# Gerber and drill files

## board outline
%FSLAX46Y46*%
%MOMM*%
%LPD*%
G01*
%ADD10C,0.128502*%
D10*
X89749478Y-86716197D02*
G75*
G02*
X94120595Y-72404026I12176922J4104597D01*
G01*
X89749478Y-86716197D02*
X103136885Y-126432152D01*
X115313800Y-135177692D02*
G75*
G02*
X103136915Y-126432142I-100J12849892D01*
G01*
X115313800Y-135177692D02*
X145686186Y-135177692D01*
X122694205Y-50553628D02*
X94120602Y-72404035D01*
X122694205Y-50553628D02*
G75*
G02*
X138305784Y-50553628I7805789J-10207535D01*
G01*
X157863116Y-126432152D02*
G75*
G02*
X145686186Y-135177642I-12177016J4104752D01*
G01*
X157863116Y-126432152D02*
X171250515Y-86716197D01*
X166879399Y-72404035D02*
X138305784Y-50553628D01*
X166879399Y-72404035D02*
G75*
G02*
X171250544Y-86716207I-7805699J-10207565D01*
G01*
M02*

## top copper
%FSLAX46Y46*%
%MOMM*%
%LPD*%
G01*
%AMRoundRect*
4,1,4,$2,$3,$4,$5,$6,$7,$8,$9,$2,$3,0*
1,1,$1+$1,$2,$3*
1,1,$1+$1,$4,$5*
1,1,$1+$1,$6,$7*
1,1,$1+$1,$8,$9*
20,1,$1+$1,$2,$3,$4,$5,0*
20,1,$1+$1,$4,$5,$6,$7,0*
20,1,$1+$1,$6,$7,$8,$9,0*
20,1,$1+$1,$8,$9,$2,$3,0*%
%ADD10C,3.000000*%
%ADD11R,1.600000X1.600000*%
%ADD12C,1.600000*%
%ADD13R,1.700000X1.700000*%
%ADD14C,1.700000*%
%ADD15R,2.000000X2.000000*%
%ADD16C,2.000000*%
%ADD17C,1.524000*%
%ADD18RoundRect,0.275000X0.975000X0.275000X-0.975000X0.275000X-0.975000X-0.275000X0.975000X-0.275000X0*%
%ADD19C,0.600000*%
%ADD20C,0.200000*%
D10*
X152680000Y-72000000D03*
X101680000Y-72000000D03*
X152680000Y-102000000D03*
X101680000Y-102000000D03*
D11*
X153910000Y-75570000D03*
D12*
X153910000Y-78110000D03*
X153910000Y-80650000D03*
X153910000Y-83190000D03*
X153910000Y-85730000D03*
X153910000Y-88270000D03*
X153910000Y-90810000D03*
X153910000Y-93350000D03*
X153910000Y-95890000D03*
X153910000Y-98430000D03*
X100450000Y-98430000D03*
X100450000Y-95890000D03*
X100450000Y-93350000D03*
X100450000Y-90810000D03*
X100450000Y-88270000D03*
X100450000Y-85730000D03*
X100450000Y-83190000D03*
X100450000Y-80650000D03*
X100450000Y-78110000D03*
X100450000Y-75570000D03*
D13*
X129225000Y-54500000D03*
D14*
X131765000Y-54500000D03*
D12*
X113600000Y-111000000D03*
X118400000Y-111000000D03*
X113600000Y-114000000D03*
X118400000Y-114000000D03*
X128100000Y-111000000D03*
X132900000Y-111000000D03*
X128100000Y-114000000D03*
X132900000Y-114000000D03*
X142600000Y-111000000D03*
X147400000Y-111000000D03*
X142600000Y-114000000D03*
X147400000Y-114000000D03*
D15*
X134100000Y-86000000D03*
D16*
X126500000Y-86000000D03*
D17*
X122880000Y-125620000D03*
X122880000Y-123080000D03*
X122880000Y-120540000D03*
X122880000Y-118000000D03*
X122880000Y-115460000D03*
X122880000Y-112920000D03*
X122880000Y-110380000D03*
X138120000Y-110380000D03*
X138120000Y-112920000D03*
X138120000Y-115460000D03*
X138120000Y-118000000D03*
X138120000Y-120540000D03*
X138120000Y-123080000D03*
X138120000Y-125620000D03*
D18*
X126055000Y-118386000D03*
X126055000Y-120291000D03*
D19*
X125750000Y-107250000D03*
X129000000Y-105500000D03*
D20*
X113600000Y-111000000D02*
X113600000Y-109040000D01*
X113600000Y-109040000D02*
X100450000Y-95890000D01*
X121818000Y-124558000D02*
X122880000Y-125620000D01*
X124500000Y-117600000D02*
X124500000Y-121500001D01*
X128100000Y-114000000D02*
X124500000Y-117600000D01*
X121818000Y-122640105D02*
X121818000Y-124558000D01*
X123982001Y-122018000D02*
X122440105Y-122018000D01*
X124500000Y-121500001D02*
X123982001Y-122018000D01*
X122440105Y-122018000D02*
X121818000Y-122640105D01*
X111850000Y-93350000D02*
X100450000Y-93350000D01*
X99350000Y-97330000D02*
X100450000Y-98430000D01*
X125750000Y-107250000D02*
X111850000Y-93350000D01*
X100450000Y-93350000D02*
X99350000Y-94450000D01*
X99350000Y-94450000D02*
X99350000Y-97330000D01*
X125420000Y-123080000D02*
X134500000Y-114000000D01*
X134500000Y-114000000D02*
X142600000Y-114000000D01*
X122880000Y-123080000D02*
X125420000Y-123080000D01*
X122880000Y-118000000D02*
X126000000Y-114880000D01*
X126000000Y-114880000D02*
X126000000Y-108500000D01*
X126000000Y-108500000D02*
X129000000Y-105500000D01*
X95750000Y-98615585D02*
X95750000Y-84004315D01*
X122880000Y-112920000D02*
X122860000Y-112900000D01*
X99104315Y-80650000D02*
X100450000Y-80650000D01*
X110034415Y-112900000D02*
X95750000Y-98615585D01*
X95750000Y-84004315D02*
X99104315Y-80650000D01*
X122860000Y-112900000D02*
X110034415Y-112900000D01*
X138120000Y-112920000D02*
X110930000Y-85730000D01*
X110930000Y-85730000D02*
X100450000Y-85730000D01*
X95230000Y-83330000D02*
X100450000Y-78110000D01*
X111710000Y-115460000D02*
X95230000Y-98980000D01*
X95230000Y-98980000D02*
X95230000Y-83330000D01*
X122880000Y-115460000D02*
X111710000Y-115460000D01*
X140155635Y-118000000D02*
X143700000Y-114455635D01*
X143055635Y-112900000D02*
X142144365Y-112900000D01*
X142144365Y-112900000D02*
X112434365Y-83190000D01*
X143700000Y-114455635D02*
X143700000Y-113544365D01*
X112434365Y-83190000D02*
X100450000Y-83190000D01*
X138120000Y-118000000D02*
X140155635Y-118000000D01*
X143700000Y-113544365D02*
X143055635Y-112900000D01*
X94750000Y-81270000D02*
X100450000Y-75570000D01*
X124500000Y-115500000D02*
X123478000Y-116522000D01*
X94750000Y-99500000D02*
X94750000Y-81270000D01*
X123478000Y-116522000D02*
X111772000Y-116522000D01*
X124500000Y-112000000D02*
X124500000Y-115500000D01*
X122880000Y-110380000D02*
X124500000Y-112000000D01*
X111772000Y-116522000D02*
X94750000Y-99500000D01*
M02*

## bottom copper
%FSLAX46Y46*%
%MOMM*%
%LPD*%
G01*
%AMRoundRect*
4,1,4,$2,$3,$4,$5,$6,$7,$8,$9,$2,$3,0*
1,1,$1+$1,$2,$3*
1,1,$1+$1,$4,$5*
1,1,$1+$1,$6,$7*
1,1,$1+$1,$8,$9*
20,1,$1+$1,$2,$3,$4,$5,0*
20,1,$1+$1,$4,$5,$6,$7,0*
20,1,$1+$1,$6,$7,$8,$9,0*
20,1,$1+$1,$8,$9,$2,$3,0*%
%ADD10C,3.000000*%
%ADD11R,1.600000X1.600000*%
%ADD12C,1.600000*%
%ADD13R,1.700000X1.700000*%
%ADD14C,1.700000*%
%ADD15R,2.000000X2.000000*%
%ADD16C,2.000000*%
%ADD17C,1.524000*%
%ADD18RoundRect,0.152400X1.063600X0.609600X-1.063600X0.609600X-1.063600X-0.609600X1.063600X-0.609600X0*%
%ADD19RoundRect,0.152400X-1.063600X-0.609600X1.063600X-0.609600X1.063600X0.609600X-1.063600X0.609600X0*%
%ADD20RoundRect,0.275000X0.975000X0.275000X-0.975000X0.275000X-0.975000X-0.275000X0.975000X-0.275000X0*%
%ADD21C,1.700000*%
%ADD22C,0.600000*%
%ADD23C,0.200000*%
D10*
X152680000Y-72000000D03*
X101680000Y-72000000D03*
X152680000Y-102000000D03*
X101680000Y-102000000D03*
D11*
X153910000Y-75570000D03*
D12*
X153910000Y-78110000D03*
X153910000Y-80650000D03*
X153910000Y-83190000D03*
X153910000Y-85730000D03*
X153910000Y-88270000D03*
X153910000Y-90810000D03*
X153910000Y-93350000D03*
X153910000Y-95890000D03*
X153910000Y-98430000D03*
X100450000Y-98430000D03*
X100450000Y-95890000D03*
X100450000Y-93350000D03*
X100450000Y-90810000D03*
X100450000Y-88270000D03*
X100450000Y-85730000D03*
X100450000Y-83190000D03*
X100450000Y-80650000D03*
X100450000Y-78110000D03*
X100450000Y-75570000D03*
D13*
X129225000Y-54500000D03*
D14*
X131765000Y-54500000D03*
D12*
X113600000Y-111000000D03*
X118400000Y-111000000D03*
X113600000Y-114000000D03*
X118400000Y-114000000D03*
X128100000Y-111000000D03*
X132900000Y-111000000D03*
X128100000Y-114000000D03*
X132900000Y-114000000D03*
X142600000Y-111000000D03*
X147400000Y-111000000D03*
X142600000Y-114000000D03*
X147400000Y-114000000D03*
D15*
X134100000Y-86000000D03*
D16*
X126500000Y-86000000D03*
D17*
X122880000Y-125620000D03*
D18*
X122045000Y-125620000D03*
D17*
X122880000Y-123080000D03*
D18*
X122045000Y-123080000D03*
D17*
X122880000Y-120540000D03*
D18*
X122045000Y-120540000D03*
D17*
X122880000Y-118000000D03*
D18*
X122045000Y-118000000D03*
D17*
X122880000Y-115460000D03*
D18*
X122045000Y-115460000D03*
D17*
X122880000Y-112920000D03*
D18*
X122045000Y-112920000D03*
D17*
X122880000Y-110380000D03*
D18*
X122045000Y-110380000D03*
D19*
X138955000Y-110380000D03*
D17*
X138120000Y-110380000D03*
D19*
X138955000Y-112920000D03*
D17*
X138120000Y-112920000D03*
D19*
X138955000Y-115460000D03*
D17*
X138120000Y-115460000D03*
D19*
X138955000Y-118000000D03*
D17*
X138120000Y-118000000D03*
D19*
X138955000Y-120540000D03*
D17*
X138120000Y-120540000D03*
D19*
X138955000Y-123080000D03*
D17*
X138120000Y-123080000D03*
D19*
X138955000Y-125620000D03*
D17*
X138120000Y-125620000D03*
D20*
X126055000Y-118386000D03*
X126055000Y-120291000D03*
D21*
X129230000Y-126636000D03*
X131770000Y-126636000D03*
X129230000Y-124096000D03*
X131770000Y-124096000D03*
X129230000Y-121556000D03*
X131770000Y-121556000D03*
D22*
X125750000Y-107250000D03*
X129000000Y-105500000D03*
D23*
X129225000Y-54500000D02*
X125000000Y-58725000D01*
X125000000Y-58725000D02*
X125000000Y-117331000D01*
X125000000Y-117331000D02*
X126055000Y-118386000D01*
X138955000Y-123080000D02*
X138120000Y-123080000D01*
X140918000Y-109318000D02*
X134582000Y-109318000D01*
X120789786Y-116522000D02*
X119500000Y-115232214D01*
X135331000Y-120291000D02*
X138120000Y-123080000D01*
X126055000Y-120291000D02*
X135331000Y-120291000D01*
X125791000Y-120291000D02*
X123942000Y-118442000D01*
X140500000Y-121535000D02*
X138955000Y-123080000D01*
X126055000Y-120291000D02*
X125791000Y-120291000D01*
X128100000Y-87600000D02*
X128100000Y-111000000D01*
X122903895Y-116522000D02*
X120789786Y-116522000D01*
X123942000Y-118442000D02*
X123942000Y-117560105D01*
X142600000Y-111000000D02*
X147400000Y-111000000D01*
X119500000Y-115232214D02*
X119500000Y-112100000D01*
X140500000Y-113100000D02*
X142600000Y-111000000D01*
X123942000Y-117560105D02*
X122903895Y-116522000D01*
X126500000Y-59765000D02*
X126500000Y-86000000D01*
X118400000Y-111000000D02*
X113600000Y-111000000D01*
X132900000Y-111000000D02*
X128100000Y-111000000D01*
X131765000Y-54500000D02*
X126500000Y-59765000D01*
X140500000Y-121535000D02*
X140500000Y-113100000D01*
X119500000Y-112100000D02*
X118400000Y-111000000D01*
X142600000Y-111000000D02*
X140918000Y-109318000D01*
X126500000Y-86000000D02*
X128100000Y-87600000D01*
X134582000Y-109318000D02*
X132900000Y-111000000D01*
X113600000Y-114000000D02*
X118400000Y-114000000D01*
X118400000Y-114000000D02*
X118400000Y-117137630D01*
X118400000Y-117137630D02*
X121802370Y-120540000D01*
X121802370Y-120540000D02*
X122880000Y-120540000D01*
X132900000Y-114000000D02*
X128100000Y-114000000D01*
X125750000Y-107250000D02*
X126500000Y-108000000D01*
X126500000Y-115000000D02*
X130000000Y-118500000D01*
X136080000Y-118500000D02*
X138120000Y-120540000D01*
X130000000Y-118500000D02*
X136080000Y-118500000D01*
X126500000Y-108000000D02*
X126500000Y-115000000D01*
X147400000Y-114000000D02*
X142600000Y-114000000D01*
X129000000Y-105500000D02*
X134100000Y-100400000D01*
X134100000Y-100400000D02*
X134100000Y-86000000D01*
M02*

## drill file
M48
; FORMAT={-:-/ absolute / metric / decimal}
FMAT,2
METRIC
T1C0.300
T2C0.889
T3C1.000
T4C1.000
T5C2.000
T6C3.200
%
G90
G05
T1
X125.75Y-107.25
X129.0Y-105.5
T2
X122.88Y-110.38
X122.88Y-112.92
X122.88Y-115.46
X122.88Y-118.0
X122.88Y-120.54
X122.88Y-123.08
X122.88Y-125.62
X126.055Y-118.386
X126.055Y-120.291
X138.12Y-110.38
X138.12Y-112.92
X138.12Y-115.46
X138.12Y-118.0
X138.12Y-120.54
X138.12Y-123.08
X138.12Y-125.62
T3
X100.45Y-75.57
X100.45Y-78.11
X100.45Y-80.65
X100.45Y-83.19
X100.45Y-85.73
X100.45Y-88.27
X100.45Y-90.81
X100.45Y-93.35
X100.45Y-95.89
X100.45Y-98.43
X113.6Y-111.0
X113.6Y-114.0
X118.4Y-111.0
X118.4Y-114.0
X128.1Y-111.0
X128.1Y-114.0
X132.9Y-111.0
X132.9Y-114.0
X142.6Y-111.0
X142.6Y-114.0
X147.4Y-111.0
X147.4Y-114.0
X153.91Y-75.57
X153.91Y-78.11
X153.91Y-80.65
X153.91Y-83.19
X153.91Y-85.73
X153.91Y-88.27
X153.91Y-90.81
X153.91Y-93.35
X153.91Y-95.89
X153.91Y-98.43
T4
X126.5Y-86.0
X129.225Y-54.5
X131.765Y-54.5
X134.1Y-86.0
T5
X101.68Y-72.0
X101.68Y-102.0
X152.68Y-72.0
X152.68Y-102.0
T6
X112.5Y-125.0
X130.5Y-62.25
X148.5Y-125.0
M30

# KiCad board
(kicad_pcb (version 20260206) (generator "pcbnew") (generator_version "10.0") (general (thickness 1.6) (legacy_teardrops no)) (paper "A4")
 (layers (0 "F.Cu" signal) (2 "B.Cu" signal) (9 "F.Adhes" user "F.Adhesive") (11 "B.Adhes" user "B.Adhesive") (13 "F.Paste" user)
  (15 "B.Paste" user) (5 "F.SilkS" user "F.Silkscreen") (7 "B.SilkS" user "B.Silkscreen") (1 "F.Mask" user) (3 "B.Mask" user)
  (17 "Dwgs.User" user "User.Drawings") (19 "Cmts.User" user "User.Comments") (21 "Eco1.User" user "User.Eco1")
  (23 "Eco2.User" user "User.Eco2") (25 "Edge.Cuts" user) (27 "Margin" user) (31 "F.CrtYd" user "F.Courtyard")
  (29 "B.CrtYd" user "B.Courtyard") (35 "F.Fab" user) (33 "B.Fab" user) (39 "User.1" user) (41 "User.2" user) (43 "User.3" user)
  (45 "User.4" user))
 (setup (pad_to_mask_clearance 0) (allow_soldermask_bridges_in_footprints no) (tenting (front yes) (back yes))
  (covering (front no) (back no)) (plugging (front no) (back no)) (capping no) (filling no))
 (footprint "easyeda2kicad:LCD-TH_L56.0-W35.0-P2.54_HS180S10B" (layer "F.Cu") (at 127.18 87 -90)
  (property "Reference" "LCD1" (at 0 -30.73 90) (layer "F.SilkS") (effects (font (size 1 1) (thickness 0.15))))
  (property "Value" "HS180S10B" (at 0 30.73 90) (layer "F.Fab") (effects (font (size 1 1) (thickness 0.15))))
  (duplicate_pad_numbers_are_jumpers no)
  (pad "" thru_hole circle (at -15 -25.5 270) (size 3 3) (drill 2) (layers "*.Cu" "*.Mask") (remove_unused_layers no))
  (pad "" thru_hole circle (at -15 25.5 270) (size 3 3) (drill 2) (layers "*.Cu" "*.Mask") (remove_unused_layers no))
  (pad "" thru_hole circle (at 15 -25.5 270) (size 3 3) (drill 2) (layers "*.Cu" "*.Mask") (remove_unused_layers no))
  (pad "" thru_hole circle (at 15 25.5 270) (size 3 3) (drill 2) (layers "*.Cu" "*.Mask") (remove_unused_layers no))
  (pad "1" thru_hole rect (at -11.43 -26.73 270) (size 1.6 1.6) (drill 0.999998) (layers "*.Cu" "*.Mask") (remove_unused_layers no)
   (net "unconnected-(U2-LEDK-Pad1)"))
  (pad "2" thru_hole circle (at -8.89 -26.73 270) (size 1.6 1.6) (drill 0.999998) (layers "*.Cu" "*.Mask") (remove_unused_layers no)
   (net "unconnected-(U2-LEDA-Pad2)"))
  (pad "3" thru_hole circle (at -6.35 -26.73 270) (size 1.6 1.6) (drill 0.999998) (layers "*.Cu" "*.Mask") (remove_unused_layers no)
   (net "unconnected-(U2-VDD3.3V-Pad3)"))
  (pad "4" thru_hole circle (at -3.81 -26.73 270) (size 1.6 1.6) (drill 0.999998) (layers "*.Cu" "*.Mask") (remove_unused_layers no)
   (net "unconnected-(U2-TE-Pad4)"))
  (pad "5" thru_hole circle (at -1.27 -26.73 270) (size 1.6 1.6) (drill 0.999998) (layers "*.Cu" "*.Mask") (remove_unused_layers no)
   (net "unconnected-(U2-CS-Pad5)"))
  (pad "6" thru_hole circle (at 1.27 -26.73 270) (size 1.6 1.6) (drill 0.999998) (layers "*.Cu" "*.Mask") (remove_unused_layers no)
   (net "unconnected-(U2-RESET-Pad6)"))
  (pad "7" thru_hole circle (at 3.81 -26.73 270) (size 1.6 1.6) (drill 0.999998) (layers "*.Cu" "*.Mask") (remove_unused_layers no)
   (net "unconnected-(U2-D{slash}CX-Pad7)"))
  (pad "8" thru_hole circle (at 6.35 -26.73 270) (size 1.6 1.6) (drill 0.999998) (layers "*.Cu" "*.Mask") (remove_unused_layers no)
   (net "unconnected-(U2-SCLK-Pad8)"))
  (pad "9" thru_hole circle (at 8.89 -26.73 270) (size 1.6 1.6) (drill 0.999998) (layers "*.Cu" "*.Mask") (remove_unused_layers no)
   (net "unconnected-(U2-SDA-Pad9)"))
  (pad "10" thru_hole circle (at 11.43 -26.73 270) (size 1.6 1.6) (drill 0.999998) (layers "*.Cu" "*.Mask") (remove_unused_layers no)
   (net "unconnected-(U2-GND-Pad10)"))
  (pad "11" thru_hole circle (at 11.43 26.73 270) (size 1.6 1.6) (drill 0.999998) (layers "*.Cu" "*.Mask") (remove_unused_layers no)
   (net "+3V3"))
  (pad "12" thru_hole circle (at 8.89 26.73 270) (size 1.6 1.6) (drill 0.999998) (layers "*.Cu" "*.Mask") (remove_unused_layers no)
   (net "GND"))
  (pad "13" thru_hole circle (at 6.35 26.73 270) (size 1.6 1.6) (drill 0.999998) (layers "*.Cu" "*.Mask") (remove_unused_layers no)
   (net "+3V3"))
  (pad "14" thru_hole circle (at 3.81 26.73 270) (size 1.6 1.6) (drill 0.999998) (layers "*.Cu" "*.Mask") (remove_unused_layers no))
  (pad "15" thru_hole circle (at 1.27 26.73 270) (size 1.6 1.6) (drill 0.999998) (layers "*.Cu" "*.Mask") (remove_unused_layers no))
  (pad "16" thru_hole circle (at -1.27 26.73 270) (size 1.6 1.6) (drill 0.999998) (layers "*.Cu" "*.Mask") (remove_unused_layers no)
   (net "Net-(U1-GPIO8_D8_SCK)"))
  (pad "17" thru_hole circle (at -3.81 26.73 270) (size 1.6 1.6) (drill 0.999998) (layers "*.Cu" "*.Mask") (remove_unused_layers no)
   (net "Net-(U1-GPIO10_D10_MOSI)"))
  (pad "18" thru_hole circle (at -6.35 26.73 270) (size 1.6 1.6) (drill 0.999998) (layers "*.Cu" "*.Mask") (remove_unused_layers no)
   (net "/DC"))
  (pad "19" thru_hole circle (at -8.89 26.73 270) (size 1.6 1.6) (drill 0.999998) (layers "*.Cu" "*.Mask") (remove_unused_layers no)
   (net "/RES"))
  (pad "20" thru_hole circle (at -11.43 26.73 270) (size 1.6 1.6) (drill 0.999998) (layers "*.Cu" "*.Mask") (remove_unused_layers no)
   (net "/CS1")))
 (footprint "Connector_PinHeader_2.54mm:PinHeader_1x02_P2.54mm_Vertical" (layer "F.Cu") (at 129.225 54.5 90)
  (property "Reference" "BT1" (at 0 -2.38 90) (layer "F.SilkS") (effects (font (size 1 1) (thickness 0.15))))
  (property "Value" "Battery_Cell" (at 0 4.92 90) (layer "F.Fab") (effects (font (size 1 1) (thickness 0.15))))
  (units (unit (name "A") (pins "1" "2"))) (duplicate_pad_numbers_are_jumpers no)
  (pad "1" thru_hole rect (at 0 0 90) (size 1.7 1.7) (drill 1) (layers "*.Cu" "*.Mask") (remove_unused_layers no) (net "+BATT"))
  (pad "2" thru_hole circle (at 0 2.54 90) (size 1.7 1.7) (drill 1) (layers "*.Cu" "*.Mask") (remove_unused_layers no) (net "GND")))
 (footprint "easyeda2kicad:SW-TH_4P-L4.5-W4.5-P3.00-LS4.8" (layer "F.Cu") (at 116 112.5)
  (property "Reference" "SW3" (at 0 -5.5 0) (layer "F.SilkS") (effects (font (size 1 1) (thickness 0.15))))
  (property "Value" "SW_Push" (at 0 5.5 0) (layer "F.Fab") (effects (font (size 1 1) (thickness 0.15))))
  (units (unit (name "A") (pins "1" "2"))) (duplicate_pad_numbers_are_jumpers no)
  (pad "1" thru_hole circle (at -2.4 -1.5) (size 1.6 1.6) (drill 0.999998) (layers "*.Cu" "*.Mask") (remove_unused_layers no) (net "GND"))
  (pad "1" thru_hole circle (at 2.4 -1.5) (size 1.6 1.6) (drill 0.999998) (layers "*.Cu" "*.Mask") (remove_unused_layers no) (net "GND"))
  (pad "2" thru_hole circle (at -2.4 1.5) (size 1.6 1.6) (drill 0.999998) (layers "*.Cu" "*.Mask") (remove_unused_layers no)
   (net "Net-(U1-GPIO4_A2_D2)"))
  (pad "2" thru_hole circle (at 2.4 1.5) (size 1.6 1.6) (drill 0.999998) (layers "*.Cu" "*.Mask") (remove_unused_layers no)
   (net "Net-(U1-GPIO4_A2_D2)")))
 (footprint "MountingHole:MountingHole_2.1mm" (layer "F.Cu") (at 148.5 125)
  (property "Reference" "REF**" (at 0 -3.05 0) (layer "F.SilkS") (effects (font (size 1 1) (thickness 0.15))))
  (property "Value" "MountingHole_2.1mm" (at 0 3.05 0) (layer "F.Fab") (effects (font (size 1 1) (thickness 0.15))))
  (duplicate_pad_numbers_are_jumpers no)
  (pad "" np_thru_hole circle (at 0 0) (size 3.2 3.2) (drill 3.2) (layers "*.Cu" "*.Mask")))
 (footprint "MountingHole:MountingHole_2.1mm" (layer "F.Cu") (at 112.5 125)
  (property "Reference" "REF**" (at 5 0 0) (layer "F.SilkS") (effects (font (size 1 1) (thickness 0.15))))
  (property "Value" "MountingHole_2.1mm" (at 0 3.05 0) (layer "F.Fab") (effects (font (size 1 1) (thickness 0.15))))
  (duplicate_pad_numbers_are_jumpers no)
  (pad "" np_thru_hole circle (at 0 0) (size 3.2 3.2) (drill 3.2) (layers "*.Cu" "*.Mask")))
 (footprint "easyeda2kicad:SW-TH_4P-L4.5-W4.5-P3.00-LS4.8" (layer "F.Cu") (at 130.5 112.5)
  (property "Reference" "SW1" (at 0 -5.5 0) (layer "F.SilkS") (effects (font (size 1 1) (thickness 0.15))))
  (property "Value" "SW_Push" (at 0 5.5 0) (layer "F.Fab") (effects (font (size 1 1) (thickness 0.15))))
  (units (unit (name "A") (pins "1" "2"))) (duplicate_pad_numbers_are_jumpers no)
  (pad "1" thru_hole circle (at -2.4 -1.5) (size 1.6 1.6) (drill 0.999998) (layers "*.Cu" "*.Mask") (remove_unused_layers no) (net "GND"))
  (pad "1" thru_hole circle (at 2.4 -1.5) (size 1.6 1.6) (drill 0.999998) (layers "*.Cu" "*.Mask") (remove_unused_layers no) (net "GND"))
  (pad "2" thru_hole circle (at -2.4 1.5) (size 1.6 1.6) (drill 0.999998) (layers "*.Cu" "*.Mask") (remove_unused_layers no)
   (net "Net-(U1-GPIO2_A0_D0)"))
  (pad "2" thru_hole circle (at 2.4 1.5) (size 1.6 1.6) (drill 0.999998) (layers "*.Cu" "*.Mask") (remove_unused_layers no)
   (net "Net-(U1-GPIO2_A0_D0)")))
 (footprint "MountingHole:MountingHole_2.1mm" (layer "F.Cu") (at 130.5 62.25)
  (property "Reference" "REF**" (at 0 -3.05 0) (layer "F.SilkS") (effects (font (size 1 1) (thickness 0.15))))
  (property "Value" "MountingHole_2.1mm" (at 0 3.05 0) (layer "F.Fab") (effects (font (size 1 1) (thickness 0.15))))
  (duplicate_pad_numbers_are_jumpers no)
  (pad "" np_thru_hole circle (at 0 0) (size 3.2 3.2) (drill 3.2) (layers "*.Cu" "*.Mask")))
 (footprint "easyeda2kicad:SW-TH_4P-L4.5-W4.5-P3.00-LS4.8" (layer "F.Cu") (at 145 112.5)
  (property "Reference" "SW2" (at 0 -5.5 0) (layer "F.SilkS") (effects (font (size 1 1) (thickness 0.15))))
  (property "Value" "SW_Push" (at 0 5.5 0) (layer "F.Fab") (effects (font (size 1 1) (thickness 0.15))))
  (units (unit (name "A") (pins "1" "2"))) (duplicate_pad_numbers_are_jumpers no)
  (pad "1" thru_hole circle (at -2.4 -1.5) (size 1.6 1.6) (drill 0.999998) (layers "*.Cu" "*.Mask") (remove_unused_layers no) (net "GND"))
  (pad "1" thru_hole circle (at 2.4 -1.5) (size 1.6 1.6) (drill 0.999998) (layers "*.Cu" "*.Mask") (remove_unused_layers no) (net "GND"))
  (pad "2" thru_hole circle (at -2.4 1.5) (size 1.6 1.6) (drill 0.999998) (layers "*.Cu" "*.Mask") (remove_unused_layers no)
   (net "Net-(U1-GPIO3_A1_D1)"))
  (pad "2" thru_hole circle (at 2.4 1.5) (size 1.6 1.6) (drill 0.999998) (layers "*.Cu" "*.Mask") (remove_unused_layers no)
   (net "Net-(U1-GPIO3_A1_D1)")))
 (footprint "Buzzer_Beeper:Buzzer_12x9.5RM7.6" (layer "B.Cu") (at 134.1 86 180)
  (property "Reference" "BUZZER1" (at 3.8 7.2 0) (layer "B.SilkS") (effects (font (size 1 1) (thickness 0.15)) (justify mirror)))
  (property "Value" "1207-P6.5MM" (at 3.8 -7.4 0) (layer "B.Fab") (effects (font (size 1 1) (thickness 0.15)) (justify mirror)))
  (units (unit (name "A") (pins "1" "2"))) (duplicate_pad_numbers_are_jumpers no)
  (pad "1" thru_hole rect (at 0 0 180) (size 2 2) (drill 1) (layers "*.Cu" "*.Mask") (remove_unused_layers no) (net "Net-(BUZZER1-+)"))
  (pad "2" thru_hole circle (at 7.6 0 180) (size 2 2) (drill 1) (layers "*.Cu" "*.Mask") (remove_unused_layers no) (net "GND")))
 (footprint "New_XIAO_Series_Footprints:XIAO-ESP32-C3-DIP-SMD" (layer "B.Cu") (at 130.5 118 -90)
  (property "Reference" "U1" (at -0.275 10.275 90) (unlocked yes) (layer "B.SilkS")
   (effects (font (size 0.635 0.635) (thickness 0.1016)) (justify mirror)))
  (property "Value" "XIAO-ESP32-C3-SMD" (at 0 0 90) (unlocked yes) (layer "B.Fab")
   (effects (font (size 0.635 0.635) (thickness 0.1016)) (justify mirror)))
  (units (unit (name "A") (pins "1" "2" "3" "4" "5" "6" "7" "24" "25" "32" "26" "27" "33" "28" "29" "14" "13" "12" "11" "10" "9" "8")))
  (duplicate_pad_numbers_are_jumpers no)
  (pad "1" thru_hole circle (at 7.62 7.62 180) (size 1.524 1.524) (drill 0.889) (layers "*.Cu" "*.Mask") (remove_unused_layers no)
   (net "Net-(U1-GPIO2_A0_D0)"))
  (pad "1" smd roundrect (at 7.62 8.455 180) (size 2.432 1.524) (layers "B.Cu" "B.Mask") (roundrect_rratio 0.1) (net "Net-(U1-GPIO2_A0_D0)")
   (thermal_bridge_angle 45))
  (pad "2" thru_hole circle (at 5.08 7.62 180) (size 1.524 1.524) (drill 0.889) (layers "*.Cu" "*.Mask") (remove_unused_layers no)
   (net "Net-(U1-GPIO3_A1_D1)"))
  (pad "2" smd roundrect (at 5.08 8.455 180) (size 2.432 1.524) (layers "B.Cu" "B.Mask") (roundrect_rratio 0.1) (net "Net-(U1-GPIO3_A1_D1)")
   (thermal_bridge_angle 45))
  (pad "3" thru_hole circle (at 2.54 7.62 180) (size 1.524 1.524) (drill 0.889) (layers "*.Cu" "*.Mask") (remove_unused_layers no)
   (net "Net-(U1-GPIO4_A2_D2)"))
  (pad "3" smd roundrect (at 2.54 8.455 180) (size 2.432 1.524) (layers "B.Cu" "B.Mask") (roundrect_rratio 0.1) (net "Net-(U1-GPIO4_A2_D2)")
   (thermal_bridge_angle 45))
  (pad "4" thru_hole circle (at 0 7.62 180) (size 1.524 1.524) (drill 0.889) (layers "*.Cu" "*.Mask") (remove_unused_layers no)
   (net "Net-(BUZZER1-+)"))
  (pad "4" smd roundrect (at 0 8.455 180) (size 2.432 1.524) (layers "B.Cu" "B.Mask") (roundrect_rratio 0.1) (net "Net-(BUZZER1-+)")
   (thermal_bridge_angle 45))
  (pad "5" thru_hole circle (at -2.54 7.62 180) (size 1.524 1.524) (drill 0.889) (layers "*.Cu" "*.Mask") (remove_unused_layers no)
   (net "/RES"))
  (pad "5" smd roundrect (at -2.54 8.455 180) (size 2.432 1.524) (layers "B.Cu" "B.Mask") (roundrect_rratio 0.1) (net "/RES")
   (thermal_bridge_angle 45))
  (pad "6" thru_hole circle (at -5.08 7.62 180) (size 1.524 1.524) (drill 0.889) (layers "*.Cu" "*.Mask") (remove_unused_layers no)
   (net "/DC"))
  (pad "6" smd roundrect (at -5.08 8.455 180) (size 2.432 1.524) (layers "B.Cu" "B.Mask") (roundrect_rratio 0.1) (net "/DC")
   (thermal_bridge_angle 45))
  (pad "7" thru_hole circle (at -7.62 7.62 180) (size 1.524 1.524) (drill 0.889) (layers "*.Cu" "*.Mask") (remove_unused_layers no)
   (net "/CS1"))
  (pad "7" smd roundrect (at -7.62 8.455 180) (size 2.432 1.524) (layers "B.Cu" "B.Mask") (roundrect_rratio 0.1) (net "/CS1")
   (thermal_bridge_angle 45))
  (pad "8" smd roundrect (at -7.62 -8.455) (size 2.432 1.524) (layers "B.Cu" "B.Mask") (roundrect_rratio 0.1)
   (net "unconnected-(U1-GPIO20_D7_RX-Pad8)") (thermal_bridge_angle 45))
  (pad "8" thru_hole circle (at -7.62 -7.62) (size 1.524 1.524) (drill 0.889) (layers "*.Cu" "*.Mask") (remove_unused_layers no)
   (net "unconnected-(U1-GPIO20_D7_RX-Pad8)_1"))
  (pad "9" smd roundrect (at -5.08 -8.455) (size 2.432 1.524) (layers "B.Cu" "B.Mask") (roundrect_rratio 0.1) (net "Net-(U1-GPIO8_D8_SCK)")
   (thermal_bridge_angle 45))
  (pad "9" thru_hole circle (at -5.08 -7.62) (size 1.524 1.524) (drill 0.889) (layers "*.Cu" "*.Mask") (remove_unused_layers no)
   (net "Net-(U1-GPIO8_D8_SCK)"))
  (pad "10" smd roundrect (at -2.54 -8.455) (size 2.432 1.524) (layers "B.Cu" "B.Mask") (roundrect_rratio 0.1)
   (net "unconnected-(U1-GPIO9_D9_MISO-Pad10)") (thermal_bridge_angle 45))
  (pad "10" thru_hole circle (at -2.54 -7.62) (size 1.524 1.524) (drill 0.889) (layers "*.Cu" "*.Mask") (remove_unused_layers no)
   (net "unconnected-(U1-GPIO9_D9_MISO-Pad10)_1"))
  (pad "11" smd roundrect (at 0 -8.455) (size 2.432 1.524) (layers "B.Cu" "B.Mask") (roundrect_rratio 0.1) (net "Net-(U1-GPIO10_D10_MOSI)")
   (thermal_bridge_angle 45))
  (pad "11" thru_hole circle (at 0 -7.62) (size 1.524 1.524) (drill 0.889) (layers "*.Cu" "*.Mask") (remove_unused_layers no)
   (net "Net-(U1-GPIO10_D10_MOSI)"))
  (pad "12" smd roundrect (at 2.54 -8.455) (size 2.432 1.524) (layers "B.Cu" "B.Mask") (roundrect_rratio 0.1) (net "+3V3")
   (thermal_bridge_angle 45))
  (pad "12" thru_hole circle (at 2.54 -7.62) (size 1.524 1.524) (drill 0.889) (layers "*.Cu" "*.Mask") (remove_unused_layers no)
   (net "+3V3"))
  (pad "13" smd roundrect (at 5.08 -8.455) (size 2.432 1.524) (layers "B.Cu" "B.Mask") (roundrect_rratio 0.1) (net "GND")
   (thermal_bridge_angle 45))
  (pad "13" thru_hole circle (at 5.08 -7.62) (size 1.524 1.524) (drill 0.889) (layers "*.Cu" "*.Mask") (remove_unused_layers no) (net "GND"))
  (pad "14" smd roundrect (at 7.62 -8.455) (size 2.432 1.524) (layers "B.Cu" "B.Mask") (roundrect_rratio 0.1) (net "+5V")
   (thermal_bridge_angle 45))
  (pad "14" thru_hole circle (at 7.62 -7.62) (size 1.524 1.524) (drill 0.889) (layers "*.Cu" "*.Mask") (remove_unused_layers no) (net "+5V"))
  (pad "15" thru_hole roundrect (at 0.386 4.445 180) (size 2.5 1.1) (drill 0.889) (layers "*.Cu" "*.Mask") (remove_unused_layers no)
   (roundrect_rratio 0.25) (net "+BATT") (thermal_bridge_angle 45))
  (pad "16" thru_hole roundrect (at 2.291 4.445 180) (size 2.5 1.1) (drill 0.889) (layers "*.Cu" "*.Mask") (remove_unused_layers no)
   (roundrect_rratio 0.25) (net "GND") (thermal_bridge_angle 45))
  (pad "17" smd circle (at 8.636 1.27) (size 1.7 1.7) (layers "B.Cu" "B.Mask" "B.Paste"))
  (pad "18" smd circle (at 8.636 -1.27) (size 1.7 1.7) (layers "B.Cu" "B.Mask" "B.Paste"))
  (pad "19" smd circle (at 6.096 1.27) (size 1.7 1.7) (layers "B.Cu" "B.Mask" "B.Paste"))
  (pad "20" smd circle (at 6.096 -1.27) (size 1.7 1.7) (layers "B.Cu" "B.Mask" "B.Paste"))
  (pad "21" smd circle (at 3.556 1.27) (size 1.7 1.7) (layers "B.Cu" "B.Mask" "B.Paste"))
  (pad "22" smd circle (at 3.556 -1.27) (size 1.7 1.7) (layers "B.Cu" "B.Mask" "B.Paste")))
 (gr_arc (start 89.749478 86.716197) (mid 89.636692 78.858169) (end 94.120602 72.404035) (stroke (width 0.128502) (type default))
  (layer "Edge.Cuts"))
 (gr_line (start 89.749478 86.716197) (end 103.136885 126.432152) (stroke (width 0.128502) (type default)) (layer "Edge.Cuts"))
 (gr_arc (start 115.3138 135.177692) (mid 107.817744 132.764785) (end 103.136885 126.432152) (stroke (width 0.128502) (type default))
  (layer "Edge.Cuts"))
 (gr_line (start 115.3138 135.177692) (end 145.686186 135.177692) (stroke (width 0.128502) (type default)) (layer "Edge.Cuts"))
 (gr_line (start 122.694205 50.553628) (end 94.120602 72.404035) (stroke (width 0.128502) (type default)) (layer "Edge.Cuts"))
 (gr_arc (start 122.694205 50.553628) (mid 130.499996 47.9111) (end 138.305784 50.553628) (stroke (width 0.128502) (type default))
  (layer "Edge.Cuts"))
 (gr_arc (start 157.863116 126.432152) (mid 153.182199 132.764729) (end 145.686186 135.177692) (stroke (width 0.128502) (type default))
  (layer "Edge.Cuts"))
 (gr_line (start 157.863116 126.432152) (end 171.250515 86.716197) (stroke (width 0.128502) (type default)) (layer "Edge.Cuts"))
 (gr_line (start 166.879399 72.404035) (end 138.305784 50.553628) (stroke (width 0.128502) (type default)) (layer "Edge.Cuts"))
 (gr_arc (start 166.879399 72.404035) (mid 171.363322 78.858174) (end 171.250515 86.716197) (stroke (width 0.128502) (type default))
  (layer "Edge.Cuts"))
 (segment (start 129.225 54.5) (end 125 58.725) (width 0.2) (layer "B.Cu") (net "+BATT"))
 (segment (start 125 58.725) (end 125 117.331) (width 0.2) (layer "B.Cu") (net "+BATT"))
 (segment (start 125 117.331) (end 126.055 118.386) (width 0.2) (layer "B.Cu") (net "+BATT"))
 (segment (start 113.6 111) (end 113.6 109.04) (width 0.2) (layer "F.Cu") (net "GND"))
 (segment (start 113.6 109.04) (end 100.45 95.89) (width 0.2) (layer "F.Cu") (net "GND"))
 (segment (start 138.955 123.08) (end 138.12 123.08) (width 0.2) (layer "B.Cu") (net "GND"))
 (segment (start 140.918 109.318) (end 134.582 109.318) (width 0.2) (layer "B.Cu") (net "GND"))
 (segment (start 120.789786 116.522) (end 119.5 115.232214) (width 0.2) (layer "B.Cu") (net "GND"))
 (segment (start 135.331 120.291) (end 138.12 123.08) (width 0.2) (layer "B.Cu") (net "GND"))
 (segment (start 126.055 120.291) (end 135.331 120.291) (width 0.2) (layer "B.Cu") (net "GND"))
 (segment (start 125.791 120.291) (end 123.942 118.442) (width 0.2) (layer "B.Cu") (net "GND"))
 (segment (start 140.5 121.535) (end 138.955 123.08) (width 0.2) (layer "B.Cu") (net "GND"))
 (segment (start 126.055 120.291) (end 125.791 120.291) (width 0.2) (layer "B.Cu") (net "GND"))
 (segment (start 128.1 87.6) (end 128.1 111) (width 0.2) (layer "B.Cu") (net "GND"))
 (segment (start 122.903895 116.522) (end 120.789786 116.522) (width 0.2) (layer "B.Cu") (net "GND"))
 (segment (start 123.942 118.442) (end 123.942 117.560105) (width 0.2) (layer "B.Cu") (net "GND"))
 (segment (start 142.6 111) (end 147.4 111) (width 0.2) (layer "B.Cu") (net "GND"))
 (segment (start 119.5 115.232214) (end 119.5 112.1) (width 0.2) (layer "B.Cu") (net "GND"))
 (segment (start 140.5 113.1) (end 142.6 111) (width 0.2) (layer "B.Cu") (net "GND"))
 (segment (start 123.942 117.560105) (end 122.903895 116.522) (width 0.2) (layer "B.Cu") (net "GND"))
 (segment (start 126.5 59.765) (end 126.5 86) (width 0.2) (layer "B.Cu") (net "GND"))
 (segment (start 118.4 111) (end 113.6 111) (width 0.2) (layer "B.Cu") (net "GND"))
 (segment (start 132.9 111) (end 128.1 111) (width 0.2) (layer "B.Cu") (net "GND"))
 (segment (start 131.765 54.5) (end 126.5 59.765) (width 0.2) (layer "B.Cu") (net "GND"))
 (segment (start 140.5 121.535) (end 140.5 113.1) (width 0.2) (layer "B.Cu") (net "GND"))
 (segment (start 119.5 112.1) (end 118.4 111) (width 0.2) (layer "B.Cu") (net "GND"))
 (segment (start 142.6 111) (end 140.918 109.318) (width 0.2) (layer "B.Cu") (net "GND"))
 (segment (start 126.5 86) (end 128.1 87.6) (width 0.2) (layer "B.Cu") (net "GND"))
 (segment (start 134.582 109.318) (end 132.9 111) (width 0.2) (layer "B.Cu") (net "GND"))
 (segment (start 113.6 114) (end 118.4 114) (width 0.2) (layer "B.Cu") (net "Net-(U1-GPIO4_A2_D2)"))
 (segment (start 118.4 114) (end 118.4 117.13763) (width 0.2) (layer "B.Cu") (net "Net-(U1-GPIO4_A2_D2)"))
 (segment (start 118.4 117.13763) (end 121.80237 120.54) (width 0.2) (layer "B.Cu") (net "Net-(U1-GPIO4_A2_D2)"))
 (segment (start 121.80237 120.54) (end 122.88 120.54) (width 0.2) (layer "B.Cu") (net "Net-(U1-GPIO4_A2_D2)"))
 (segment (start 121.818 124.558) (end 122.88 125.62) (width 0.2) (layer "F.Cu") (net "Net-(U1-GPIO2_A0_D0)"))
 (segment (start 124.5 117.6) (end 124.5 121.500001) (width 0.2) (layer "F.Cu") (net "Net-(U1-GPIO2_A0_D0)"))
 (segment (start 128.1 114) (end 124.5 117.6) (width 0.2) (layer "F.Cu") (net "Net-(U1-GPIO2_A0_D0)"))
 (segment (start 121.818 122.640105) (end 121.818 124.558) (width 0.2) (layer "F.Cu") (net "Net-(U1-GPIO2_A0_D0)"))
 (segment (start 123.982001 122.018) (end 122.440105 122.018) (width 0.2) (layer "F.Cu") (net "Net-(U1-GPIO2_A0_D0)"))
 (segment (start 124.5 121.500001) (end 123.982001 122.018) (width 0.2) (layer "F.Cu") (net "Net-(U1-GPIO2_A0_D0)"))
 (segment (start 122.440105 122.018) (end 121.818 122.640105) (width 0.2) (layer "F.Cu") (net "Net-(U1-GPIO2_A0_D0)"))
 (segment (start 132.9 114) (end 128.1 114) (width 0.2) (layer "B.Cu") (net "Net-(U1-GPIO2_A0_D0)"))
 (segment (start 111.85 93.35) (end 100.45 93.35) (width 0.2) (layer "F.Cu") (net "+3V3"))
 (segment (start 99.35 97.33) (end 100.45 98.43) (width 0.2) (layer "F.Cu") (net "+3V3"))
 (segment (start 125.75 107.25) (end 111.85 93.35) (width 0.2) (layer "F.Cu") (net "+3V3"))
 (segment (start 100.45 93.35) (end 99.35 94.45) (width 0.2) (layer "F.Cu") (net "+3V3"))
 (segment (start 99.35 94.45) (end 99.35 97.33) (width 0.2) (layer "F.Cu") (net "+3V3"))
 (via (at 125.75 107.25) (size 0.6) (drill 0.3) (layers "F.Cu" "B.Cu") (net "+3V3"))
 (segment (start 125.75 107.25) (end 126.5 108) (width 0.2) (layer "B.Cu") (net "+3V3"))
 (segment (start 126.5 115) (end 130 118.5) (width 0.2) (layer "B.Cu") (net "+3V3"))
 (segment (start 136.08 118.5) (end 138.12 120.54) (width 0.2) (layer "B.Cu") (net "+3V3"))
 (segment (start 130 118.5) (end 136.08 118.5) (width 0.2) (layer "B.Cu") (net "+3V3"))
 (segment (start 126.5 108) (end 126.5 115) (width 0.2) (layer "B.Cu") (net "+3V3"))
 (segment (start 125.42 123.08) (end 134.5 114) (width 0.2) (layer "F.Cu") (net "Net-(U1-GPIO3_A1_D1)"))
 (segment (start 134.5 114) (end 142.6 114) (width 0.2) (layer "F.Cu") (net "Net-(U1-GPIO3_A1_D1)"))
 (segment (start 122.88 123.08) (end 125.42 123.08) (width 0.2) (layer "F.Cu") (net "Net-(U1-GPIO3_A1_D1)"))
 (segment (start 147.4 114) (end 142.6 114) (width 0.2) (layer "B.Cu") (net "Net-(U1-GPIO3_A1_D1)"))
 (segment (start 122.88 118) (end 126 114.88) (width 0.2) (layer "F.Cu") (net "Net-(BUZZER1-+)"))
 (segment (start 126 114.88) (end 126 108.5) (width 0.2) (layer "F.Cu") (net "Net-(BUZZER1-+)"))
 (segment (start 126 108.5) (end 129 105.5) (width 0.2) (layer "F.Cu") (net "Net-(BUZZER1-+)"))
 (via (at 129 105.5) (size 0.6) (drill 0.3) (layers "F.Cu" "B.Cu") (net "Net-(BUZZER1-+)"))
 (segment (start 129 105.5) (end 134.1 100.4) (width 0.2) (layer "B.Cu") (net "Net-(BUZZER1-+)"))
 (segment (start 134.1 100.4) (end 134.1 86) (width 0.2) (layer "B.Cu") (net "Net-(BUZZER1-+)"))
 (segment (start 95.75 98.615585) (end 95.75 84.004315) (width 0.2) (layer "F.Cu") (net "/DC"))
 (segment (start 122.88 112.92) (end 122.86 112.9) (width 0.2) (layer "F.Cu") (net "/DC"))
 (segment (start 99.104315 80.65) (end 100.45 80.65) (width 0.2) (layer "F.Cu") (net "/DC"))
 (segment (start 110.034415 112.9) (end 95.75 98.615585) (width 0.2) (layer "F.Cu") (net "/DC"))
 (segment (start 95.75 84.004315) (end 99.104315 80.65) (width 0.2) (layer "F.Cu") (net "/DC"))
 (segment (start 122.86 112.9) (end 110.034415 112.9) (width 0.2) (layer "F.Cu") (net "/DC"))
 (segment (start 138.12 112.92) (end 110.93 85.73) (width 0.2) (layer "F.Cu") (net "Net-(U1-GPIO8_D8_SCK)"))
 (segment (start 110.93 85.73) (end 100.45 85.73) (width 0.2) (layer "F.Cu") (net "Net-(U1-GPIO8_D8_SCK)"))
 (segment (start 95.23 83.33) (end 100.45 78.11) (width 0.2) (layer "F.Cu") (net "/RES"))
 (segment (start 111.71 115.46) (end 95.23 98.98) (width 0.2) (layer "F.Cu") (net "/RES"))
 (segment (start 95.23 98.98) (end 95.23 83.33) (width 0.2) (layer "F.Cu") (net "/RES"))
 (segment (start 122.88 115.46) (end 111.71 115.46) (width 0.2) (layer "F.Cu") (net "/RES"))
 (segment (start 140.155635 118) (end 143.7 114.455635) (width 0.2) (layer "F.Cu") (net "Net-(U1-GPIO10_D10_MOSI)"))
 (segment (start 143.055635 112.9) (end 142.144365 112.9) (width 0.2) (layer "F.Cu") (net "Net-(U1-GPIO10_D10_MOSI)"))
 (segment (start 142.144365 112.9) (end 112.434365 83.19) (width 0.2) (layer "F.Cu") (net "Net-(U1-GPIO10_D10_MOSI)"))
 (segment (start 143.7 114.455635) (end 143.7 113.544365) (width 0.2) (layer "F.Cu") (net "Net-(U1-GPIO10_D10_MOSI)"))
 (segment (start 112.434365 83.19) (end 100.45 83.19) (width 0.2) (layer "F.Cu") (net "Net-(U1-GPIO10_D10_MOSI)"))
 (segment (start 138.12 118) (end 140.155635 118) (width 0.2) (layer "F.Cu") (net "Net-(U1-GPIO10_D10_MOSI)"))
 (segment (start 143.7 113.544365) (end 143.055635 112.9) (width 0.2) (layer "F.Cu") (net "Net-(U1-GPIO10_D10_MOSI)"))
 (segment (start 94.75 81.27) (end 100.45 75.57) (width 0.2) (layer "F.Cu") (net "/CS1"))
 (segment (start 124.5 115.5) (end 123.478 116.522) (width 0.2) (layer "F.Cu") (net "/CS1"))
 (segment (start 94.75 99.5) (end 94.75 81.27) (width 0.2) (layer "F.Cu") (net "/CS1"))
 (segment (start 123.478 116.522) (end 111.772 116.522) (width 0.2) (layer "F.Cu") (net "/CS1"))
 (segment (start 124.5 112) (end 124.5 115.5) (width 0.2) (layer "F.Cu") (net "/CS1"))
 (segment (start 122.88 110.38) (end 124.5 112) (width 0.2) (layer "F.Cu") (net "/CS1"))
 (segment (start 111.772 116.522) (end 94.75 99.5) (width 0.2) (layer "F.Cu") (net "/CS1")))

